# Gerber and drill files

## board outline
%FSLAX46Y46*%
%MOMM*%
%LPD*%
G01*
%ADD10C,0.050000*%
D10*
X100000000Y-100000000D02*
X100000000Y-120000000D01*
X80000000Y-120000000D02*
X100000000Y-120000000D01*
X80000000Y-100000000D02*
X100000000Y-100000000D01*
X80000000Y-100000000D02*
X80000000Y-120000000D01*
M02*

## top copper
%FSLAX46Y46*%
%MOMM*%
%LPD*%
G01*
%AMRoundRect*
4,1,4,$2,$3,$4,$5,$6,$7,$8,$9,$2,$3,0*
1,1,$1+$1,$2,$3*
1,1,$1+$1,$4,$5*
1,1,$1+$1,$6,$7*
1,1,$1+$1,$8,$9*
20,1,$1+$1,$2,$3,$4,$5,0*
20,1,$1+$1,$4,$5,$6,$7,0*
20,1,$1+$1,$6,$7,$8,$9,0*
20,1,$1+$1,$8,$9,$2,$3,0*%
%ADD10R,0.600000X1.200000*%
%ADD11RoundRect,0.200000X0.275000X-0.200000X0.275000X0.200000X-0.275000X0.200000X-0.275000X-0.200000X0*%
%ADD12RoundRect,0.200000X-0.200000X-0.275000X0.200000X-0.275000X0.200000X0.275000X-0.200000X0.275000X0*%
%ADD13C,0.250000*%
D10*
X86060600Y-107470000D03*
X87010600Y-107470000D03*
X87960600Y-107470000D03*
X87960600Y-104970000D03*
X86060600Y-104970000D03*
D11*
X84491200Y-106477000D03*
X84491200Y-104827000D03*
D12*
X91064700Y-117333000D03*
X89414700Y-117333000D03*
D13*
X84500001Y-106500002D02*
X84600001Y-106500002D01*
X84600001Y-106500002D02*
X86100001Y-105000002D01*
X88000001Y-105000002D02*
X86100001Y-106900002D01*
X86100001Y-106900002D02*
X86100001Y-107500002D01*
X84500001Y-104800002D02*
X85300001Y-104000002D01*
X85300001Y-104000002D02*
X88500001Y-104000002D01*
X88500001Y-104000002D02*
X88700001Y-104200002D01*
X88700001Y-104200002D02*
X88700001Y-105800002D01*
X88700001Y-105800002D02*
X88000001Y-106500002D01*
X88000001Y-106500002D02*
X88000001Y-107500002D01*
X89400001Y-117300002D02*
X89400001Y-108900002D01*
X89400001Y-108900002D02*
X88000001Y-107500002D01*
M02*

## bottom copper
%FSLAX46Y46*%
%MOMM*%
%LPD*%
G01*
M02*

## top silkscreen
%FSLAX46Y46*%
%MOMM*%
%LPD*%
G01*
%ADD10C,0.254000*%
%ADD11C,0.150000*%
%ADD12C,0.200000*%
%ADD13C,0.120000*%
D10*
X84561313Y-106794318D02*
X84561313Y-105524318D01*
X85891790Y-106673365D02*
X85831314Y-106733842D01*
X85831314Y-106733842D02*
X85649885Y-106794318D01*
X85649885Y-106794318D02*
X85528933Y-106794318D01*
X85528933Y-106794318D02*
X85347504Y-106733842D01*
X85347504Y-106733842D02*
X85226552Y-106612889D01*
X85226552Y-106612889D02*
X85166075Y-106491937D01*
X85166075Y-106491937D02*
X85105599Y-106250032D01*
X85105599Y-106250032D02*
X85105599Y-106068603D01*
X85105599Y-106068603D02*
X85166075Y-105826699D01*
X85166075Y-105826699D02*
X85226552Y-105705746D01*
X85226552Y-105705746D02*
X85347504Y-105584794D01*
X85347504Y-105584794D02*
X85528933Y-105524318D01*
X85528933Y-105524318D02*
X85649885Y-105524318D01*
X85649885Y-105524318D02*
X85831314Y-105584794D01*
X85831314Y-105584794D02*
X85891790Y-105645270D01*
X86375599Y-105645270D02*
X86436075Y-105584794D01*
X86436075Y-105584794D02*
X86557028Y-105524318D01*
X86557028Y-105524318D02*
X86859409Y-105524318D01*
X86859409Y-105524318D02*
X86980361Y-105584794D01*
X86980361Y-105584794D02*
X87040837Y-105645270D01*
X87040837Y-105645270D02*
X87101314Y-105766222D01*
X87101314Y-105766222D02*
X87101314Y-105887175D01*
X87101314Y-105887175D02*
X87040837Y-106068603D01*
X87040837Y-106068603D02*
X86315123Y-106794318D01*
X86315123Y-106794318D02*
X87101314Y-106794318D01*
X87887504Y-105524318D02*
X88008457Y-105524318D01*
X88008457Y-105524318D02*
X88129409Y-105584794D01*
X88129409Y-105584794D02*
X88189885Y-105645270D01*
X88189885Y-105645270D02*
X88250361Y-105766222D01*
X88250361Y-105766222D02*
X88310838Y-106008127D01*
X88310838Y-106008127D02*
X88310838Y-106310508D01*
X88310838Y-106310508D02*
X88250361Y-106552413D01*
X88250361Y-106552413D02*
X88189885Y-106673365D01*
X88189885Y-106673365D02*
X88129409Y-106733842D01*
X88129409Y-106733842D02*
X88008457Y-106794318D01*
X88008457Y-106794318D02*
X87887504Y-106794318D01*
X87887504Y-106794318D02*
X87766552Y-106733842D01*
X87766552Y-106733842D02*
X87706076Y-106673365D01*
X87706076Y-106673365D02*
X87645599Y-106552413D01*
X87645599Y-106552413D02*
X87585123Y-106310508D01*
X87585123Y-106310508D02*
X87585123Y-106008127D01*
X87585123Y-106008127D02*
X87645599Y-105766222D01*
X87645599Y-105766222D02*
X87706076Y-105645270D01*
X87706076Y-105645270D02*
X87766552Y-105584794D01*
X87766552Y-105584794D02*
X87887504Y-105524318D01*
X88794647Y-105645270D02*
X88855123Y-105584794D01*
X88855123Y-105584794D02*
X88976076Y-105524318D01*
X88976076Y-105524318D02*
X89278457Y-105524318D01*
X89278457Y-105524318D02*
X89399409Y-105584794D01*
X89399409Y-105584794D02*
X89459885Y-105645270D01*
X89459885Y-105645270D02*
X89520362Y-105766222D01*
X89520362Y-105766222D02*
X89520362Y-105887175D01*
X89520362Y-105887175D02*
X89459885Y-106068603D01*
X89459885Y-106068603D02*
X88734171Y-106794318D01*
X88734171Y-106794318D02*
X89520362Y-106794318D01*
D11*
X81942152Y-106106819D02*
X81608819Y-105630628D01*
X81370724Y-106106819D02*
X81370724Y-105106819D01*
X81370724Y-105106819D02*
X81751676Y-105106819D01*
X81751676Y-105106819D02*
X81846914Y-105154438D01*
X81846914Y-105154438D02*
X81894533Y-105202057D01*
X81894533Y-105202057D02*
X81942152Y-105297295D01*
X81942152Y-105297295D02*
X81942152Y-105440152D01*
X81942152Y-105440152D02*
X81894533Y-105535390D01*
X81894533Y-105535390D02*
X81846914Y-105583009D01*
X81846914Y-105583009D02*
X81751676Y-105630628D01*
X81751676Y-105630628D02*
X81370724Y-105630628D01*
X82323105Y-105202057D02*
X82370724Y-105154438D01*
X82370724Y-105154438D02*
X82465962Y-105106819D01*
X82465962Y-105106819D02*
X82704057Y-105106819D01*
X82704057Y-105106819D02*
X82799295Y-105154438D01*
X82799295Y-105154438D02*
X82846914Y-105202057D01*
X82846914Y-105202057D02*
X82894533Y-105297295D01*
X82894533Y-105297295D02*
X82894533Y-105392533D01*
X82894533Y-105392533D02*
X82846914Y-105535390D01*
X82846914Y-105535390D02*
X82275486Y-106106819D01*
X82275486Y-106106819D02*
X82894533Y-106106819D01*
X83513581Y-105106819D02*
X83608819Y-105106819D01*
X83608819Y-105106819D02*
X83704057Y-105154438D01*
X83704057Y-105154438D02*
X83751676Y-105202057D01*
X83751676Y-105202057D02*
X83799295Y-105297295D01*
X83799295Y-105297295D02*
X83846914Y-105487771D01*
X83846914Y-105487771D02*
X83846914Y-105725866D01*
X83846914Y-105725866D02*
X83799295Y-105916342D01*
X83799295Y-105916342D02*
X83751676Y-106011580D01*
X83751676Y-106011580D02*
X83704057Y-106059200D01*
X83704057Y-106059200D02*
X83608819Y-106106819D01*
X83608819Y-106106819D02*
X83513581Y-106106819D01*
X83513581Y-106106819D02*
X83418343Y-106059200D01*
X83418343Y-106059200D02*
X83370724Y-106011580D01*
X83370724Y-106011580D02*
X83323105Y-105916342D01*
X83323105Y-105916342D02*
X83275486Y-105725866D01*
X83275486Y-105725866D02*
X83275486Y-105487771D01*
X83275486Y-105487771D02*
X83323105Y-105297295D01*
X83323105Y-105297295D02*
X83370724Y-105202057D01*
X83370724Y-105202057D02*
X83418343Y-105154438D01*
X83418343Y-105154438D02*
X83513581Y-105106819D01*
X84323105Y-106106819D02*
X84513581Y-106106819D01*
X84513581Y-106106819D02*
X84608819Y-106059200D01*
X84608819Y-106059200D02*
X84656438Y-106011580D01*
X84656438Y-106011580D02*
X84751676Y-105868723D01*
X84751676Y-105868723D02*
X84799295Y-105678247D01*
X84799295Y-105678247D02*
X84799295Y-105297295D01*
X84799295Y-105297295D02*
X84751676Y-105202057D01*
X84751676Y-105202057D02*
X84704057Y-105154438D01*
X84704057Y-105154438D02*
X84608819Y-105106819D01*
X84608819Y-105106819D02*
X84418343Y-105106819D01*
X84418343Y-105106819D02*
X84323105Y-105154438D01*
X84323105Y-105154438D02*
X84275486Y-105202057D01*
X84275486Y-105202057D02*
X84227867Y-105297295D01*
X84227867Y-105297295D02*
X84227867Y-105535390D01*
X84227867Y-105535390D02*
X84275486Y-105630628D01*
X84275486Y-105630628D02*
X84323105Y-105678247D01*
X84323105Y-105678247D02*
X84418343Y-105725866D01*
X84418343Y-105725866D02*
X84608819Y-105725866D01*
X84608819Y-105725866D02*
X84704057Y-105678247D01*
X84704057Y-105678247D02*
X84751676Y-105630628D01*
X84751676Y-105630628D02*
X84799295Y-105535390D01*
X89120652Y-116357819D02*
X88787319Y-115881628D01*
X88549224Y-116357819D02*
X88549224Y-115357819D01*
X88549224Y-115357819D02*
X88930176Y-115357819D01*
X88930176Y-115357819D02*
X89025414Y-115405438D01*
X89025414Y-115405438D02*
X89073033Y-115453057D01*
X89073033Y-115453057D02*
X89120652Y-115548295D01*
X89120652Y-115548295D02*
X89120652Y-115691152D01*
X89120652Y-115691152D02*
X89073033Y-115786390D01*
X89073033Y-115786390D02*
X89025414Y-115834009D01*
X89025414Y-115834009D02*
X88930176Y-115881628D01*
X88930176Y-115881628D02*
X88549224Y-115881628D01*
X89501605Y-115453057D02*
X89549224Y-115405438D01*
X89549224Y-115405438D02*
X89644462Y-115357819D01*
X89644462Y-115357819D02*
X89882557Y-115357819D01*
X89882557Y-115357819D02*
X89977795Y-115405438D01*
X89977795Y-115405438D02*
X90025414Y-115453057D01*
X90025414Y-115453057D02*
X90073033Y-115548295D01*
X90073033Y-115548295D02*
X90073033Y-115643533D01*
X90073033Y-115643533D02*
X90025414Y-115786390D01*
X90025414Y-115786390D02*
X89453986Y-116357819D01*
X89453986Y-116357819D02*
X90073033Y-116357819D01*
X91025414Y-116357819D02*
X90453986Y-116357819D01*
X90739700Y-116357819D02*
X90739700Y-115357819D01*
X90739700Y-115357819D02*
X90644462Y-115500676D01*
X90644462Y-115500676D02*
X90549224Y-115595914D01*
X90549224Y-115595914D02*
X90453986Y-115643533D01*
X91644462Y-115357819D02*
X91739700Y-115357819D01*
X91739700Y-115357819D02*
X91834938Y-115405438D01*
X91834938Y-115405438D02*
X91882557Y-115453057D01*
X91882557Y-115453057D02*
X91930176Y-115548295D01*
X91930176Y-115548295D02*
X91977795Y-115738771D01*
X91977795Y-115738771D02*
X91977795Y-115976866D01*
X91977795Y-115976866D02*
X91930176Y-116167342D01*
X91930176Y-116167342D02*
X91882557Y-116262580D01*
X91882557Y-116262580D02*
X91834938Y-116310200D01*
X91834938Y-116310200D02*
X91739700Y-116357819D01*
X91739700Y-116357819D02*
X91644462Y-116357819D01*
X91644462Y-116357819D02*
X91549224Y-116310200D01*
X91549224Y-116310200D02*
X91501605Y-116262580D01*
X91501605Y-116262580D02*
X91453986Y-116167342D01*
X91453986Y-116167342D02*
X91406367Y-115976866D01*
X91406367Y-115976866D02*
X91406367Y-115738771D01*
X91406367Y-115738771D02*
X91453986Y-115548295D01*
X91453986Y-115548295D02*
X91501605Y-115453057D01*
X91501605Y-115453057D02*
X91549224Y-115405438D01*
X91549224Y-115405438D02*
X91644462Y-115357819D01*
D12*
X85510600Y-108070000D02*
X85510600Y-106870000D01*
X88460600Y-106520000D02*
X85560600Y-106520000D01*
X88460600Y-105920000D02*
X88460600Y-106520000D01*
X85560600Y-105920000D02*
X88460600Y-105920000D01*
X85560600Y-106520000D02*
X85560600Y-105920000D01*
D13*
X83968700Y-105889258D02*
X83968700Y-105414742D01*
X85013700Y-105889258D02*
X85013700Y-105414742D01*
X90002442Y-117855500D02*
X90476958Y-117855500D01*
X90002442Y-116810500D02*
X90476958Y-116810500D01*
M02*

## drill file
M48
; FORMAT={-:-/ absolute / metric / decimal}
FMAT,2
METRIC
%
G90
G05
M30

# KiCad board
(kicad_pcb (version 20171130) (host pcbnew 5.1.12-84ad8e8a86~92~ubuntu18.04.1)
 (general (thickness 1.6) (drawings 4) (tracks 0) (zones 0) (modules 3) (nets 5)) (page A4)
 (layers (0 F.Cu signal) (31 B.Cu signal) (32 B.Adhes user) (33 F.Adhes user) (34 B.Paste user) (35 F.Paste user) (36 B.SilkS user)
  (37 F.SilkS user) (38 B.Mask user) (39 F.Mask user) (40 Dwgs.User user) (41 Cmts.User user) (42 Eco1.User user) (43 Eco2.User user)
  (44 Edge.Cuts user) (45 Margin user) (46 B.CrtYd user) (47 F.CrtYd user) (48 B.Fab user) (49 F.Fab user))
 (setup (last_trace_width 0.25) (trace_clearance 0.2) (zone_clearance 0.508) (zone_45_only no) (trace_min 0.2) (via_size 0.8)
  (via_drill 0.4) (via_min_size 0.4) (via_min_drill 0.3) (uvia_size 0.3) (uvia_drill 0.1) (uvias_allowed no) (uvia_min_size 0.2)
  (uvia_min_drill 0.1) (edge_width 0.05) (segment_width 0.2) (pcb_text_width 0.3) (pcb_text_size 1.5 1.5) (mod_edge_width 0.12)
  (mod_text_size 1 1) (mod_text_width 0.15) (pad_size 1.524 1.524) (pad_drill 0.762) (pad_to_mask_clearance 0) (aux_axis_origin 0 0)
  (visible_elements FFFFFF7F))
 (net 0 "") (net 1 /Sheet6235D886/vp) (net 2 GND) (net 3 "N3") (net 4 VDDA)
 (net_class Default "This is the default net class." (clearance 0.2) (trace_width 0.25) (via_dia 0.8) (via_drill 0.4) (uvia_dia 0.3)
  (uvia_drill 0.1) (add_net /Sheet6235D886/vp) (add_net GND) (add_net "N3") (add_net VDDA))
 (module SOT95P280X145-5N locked (layer F.Cu) (at 87.010600 106.220000 90.000000)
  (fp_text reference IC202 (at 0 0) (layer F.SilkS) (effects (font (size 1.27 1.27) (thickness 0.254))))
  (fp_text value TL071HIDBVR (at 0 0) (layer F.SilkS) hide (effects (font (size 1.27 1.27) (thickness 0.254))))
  (fp_line (start -1.85 -1.5) (end -0.65 -1.5) (layer F.SilkS) (width 0.2))
  (fp_line (start -0.3 1.45) (end -0.3 -1.45) (layer F.SilkS) (width 0.2))
  (fp_line (start 0.3 1.45) (end -0.3 1.45) (layer F.SilkS) (width 0.2))
  (fp_line (start 0.3 -1.45) (end 0.3 1.45) (layer F.SilkS) (width 0.2))
  (fp_line (start -0.3 -1.45) (end 0.3 -1.45) (layer F.SilkS) (width 0.2))
  (pad 1 smd rect (at -1.25 -0.95 180.000000) (size 0.6 1.2) (layers F.Cu F.Mask F.Paste) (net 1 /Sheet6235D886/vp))
  (pad 2 smd rect (at -1.25 0 180.000000) (size 0.6 1.2) (layers F.Cu F.Mask F.Paste) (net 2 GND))
  (pad 3 smd rect (at -1.25 0.95 180.000000) (size 0.6 1.2) (layers F.Cu F.Mask F.Paste) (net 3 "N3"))
  (pad 4 smd rect (at 1.25 0.95 180.000000) (size 0.6 1.2) (layers F.Cu F.Mask F.Paste) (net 1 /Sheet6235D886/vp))
  (pad 5 smd rect (at 1.25 -0.95 180.000000) (size 0.6 1.2) (layers F.Cu F.Mask F.Paste) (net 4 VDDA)))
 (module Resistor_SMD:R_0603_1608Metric (layer F.Cu) (at 84.491200 105.652000 90.000000)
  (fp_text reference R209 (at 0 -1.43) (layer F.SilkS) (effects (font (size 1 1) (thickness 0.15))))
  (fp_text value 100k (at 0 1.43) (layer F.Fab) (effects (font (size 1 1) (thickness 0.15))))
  (fp_line (start -0.237258 -0.5225) (end 0.237258 -0.5225) (layer F.SilkS) (width 0.12))
  (fp_line (start -0.237258 0.5225) (end 0.237258 0.5225) (layer F.SilkS) (width 0.12))
  (pad 1 smd roundrect (at -0.825 0 90.000000) (size 0.8 0.95) (layers F.Cu F.Mask F.Paste) (roundrect_rratio 0.25) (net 4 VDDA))
  (pad 2 smd roundrect (at 0.825 0 90.000000) (size 0.8 0.95) (layers F.Cu F.Mask F.Paste) (roundrect_rratio 0.25) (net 3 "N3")))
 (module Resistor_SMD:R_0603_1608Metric (layer F.Cu) (at 90.239700 117.333000)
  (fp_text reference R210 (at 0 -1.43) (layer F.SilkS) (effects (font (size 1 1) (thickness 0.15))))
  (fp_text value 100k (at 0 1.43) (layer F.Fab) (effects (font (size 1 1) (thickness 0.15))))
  (fp_line (start -0.237258 0.5225) (end 0.237258 0.5225) (layer F.SilkS) (width 0.12))
  (fp_line (start -0.237258 -0.5225) (end 0.237258 -0.5225) (layer F.SilkS) (width 0.12))
  (pad 2 smd roundrect (at 0.825 0) (size 0.8 0.95) (layers F.Cu F.Mask F.Paste) (roundrect_rratio 0.25) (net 2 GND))
  (pad 1 smd roundrect (at -0.825 0) (size 0.8 0.95) (layers F.Cu F.Mask F.Paste) (roundrect_rratio 0.25) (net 3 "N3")))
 (gr_line (start 100 100) (end 100 120) (layer Edge.Cuts) (width 0.05))
 (gr_line (start 80 120) (end 100 120) (layer Edge.Cuts) (width 0.05))
 (gr_line (start 80 100) (end 100 100) (layer Edge.Cuts) (width 0.05))
 (gr_line (start 80 100) (end 80 120) (layer Edge.Cuts) (width 0.05))
 (segment (start 84.500001 106.500002) (end 84.600001 106.500002) (width 0.250000) (layer F.Cu) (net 4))
 (segment (start 84.600001 106.500002) (end 86.100001 105.000002) (width 0.250000) (layer F.Cu) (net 4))
 (segment (start 88.000001 105.000002) (end 86.100001 106.900002) (width 0.250000) (layer F.Cu) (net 1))
 (segment (start 86.100001 106.900002) (end 86.100001 107.500002) (width 0.250000) (layer F.Cu) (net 1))
 (segment (start 84.500001 104.800002) (end 85.300001 104.000002) (width 0.250000) (layer F.Cu) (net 3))
 (segment (start 85.300001 104.000002) (end 88.500001 104.000002) (width 0.250000) (layer F.Cu) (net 3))
 (segment (start 88.500001 104.000002) (end 88.700001 104.200002) (width 0.250000) (layer F.Cu) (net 3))
 (segment (start 88.700001 104.200002) (end 88.700001 105.800002) (width 0.250000) (layer F.Cu) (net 3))
 (segment (start 88.700001 105.800002) (end 88.000001 106.500002) (width 0.250000) (layer F.Cu) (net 3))
 (segment (start 88.000001 106.500002) (end 88.000001 107.500002) (width 0.250000) (layer F.Cu) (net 3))
 (segment (start 89.400001 117.300002) (end 89.400001 108.900002) (width 0.250000) (layer F.Cu) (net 3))
 (segment (start 89.400001 108.900002) (end 88.000001 107.500002) (width 0.250000) (layer F.Cu) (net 3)))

